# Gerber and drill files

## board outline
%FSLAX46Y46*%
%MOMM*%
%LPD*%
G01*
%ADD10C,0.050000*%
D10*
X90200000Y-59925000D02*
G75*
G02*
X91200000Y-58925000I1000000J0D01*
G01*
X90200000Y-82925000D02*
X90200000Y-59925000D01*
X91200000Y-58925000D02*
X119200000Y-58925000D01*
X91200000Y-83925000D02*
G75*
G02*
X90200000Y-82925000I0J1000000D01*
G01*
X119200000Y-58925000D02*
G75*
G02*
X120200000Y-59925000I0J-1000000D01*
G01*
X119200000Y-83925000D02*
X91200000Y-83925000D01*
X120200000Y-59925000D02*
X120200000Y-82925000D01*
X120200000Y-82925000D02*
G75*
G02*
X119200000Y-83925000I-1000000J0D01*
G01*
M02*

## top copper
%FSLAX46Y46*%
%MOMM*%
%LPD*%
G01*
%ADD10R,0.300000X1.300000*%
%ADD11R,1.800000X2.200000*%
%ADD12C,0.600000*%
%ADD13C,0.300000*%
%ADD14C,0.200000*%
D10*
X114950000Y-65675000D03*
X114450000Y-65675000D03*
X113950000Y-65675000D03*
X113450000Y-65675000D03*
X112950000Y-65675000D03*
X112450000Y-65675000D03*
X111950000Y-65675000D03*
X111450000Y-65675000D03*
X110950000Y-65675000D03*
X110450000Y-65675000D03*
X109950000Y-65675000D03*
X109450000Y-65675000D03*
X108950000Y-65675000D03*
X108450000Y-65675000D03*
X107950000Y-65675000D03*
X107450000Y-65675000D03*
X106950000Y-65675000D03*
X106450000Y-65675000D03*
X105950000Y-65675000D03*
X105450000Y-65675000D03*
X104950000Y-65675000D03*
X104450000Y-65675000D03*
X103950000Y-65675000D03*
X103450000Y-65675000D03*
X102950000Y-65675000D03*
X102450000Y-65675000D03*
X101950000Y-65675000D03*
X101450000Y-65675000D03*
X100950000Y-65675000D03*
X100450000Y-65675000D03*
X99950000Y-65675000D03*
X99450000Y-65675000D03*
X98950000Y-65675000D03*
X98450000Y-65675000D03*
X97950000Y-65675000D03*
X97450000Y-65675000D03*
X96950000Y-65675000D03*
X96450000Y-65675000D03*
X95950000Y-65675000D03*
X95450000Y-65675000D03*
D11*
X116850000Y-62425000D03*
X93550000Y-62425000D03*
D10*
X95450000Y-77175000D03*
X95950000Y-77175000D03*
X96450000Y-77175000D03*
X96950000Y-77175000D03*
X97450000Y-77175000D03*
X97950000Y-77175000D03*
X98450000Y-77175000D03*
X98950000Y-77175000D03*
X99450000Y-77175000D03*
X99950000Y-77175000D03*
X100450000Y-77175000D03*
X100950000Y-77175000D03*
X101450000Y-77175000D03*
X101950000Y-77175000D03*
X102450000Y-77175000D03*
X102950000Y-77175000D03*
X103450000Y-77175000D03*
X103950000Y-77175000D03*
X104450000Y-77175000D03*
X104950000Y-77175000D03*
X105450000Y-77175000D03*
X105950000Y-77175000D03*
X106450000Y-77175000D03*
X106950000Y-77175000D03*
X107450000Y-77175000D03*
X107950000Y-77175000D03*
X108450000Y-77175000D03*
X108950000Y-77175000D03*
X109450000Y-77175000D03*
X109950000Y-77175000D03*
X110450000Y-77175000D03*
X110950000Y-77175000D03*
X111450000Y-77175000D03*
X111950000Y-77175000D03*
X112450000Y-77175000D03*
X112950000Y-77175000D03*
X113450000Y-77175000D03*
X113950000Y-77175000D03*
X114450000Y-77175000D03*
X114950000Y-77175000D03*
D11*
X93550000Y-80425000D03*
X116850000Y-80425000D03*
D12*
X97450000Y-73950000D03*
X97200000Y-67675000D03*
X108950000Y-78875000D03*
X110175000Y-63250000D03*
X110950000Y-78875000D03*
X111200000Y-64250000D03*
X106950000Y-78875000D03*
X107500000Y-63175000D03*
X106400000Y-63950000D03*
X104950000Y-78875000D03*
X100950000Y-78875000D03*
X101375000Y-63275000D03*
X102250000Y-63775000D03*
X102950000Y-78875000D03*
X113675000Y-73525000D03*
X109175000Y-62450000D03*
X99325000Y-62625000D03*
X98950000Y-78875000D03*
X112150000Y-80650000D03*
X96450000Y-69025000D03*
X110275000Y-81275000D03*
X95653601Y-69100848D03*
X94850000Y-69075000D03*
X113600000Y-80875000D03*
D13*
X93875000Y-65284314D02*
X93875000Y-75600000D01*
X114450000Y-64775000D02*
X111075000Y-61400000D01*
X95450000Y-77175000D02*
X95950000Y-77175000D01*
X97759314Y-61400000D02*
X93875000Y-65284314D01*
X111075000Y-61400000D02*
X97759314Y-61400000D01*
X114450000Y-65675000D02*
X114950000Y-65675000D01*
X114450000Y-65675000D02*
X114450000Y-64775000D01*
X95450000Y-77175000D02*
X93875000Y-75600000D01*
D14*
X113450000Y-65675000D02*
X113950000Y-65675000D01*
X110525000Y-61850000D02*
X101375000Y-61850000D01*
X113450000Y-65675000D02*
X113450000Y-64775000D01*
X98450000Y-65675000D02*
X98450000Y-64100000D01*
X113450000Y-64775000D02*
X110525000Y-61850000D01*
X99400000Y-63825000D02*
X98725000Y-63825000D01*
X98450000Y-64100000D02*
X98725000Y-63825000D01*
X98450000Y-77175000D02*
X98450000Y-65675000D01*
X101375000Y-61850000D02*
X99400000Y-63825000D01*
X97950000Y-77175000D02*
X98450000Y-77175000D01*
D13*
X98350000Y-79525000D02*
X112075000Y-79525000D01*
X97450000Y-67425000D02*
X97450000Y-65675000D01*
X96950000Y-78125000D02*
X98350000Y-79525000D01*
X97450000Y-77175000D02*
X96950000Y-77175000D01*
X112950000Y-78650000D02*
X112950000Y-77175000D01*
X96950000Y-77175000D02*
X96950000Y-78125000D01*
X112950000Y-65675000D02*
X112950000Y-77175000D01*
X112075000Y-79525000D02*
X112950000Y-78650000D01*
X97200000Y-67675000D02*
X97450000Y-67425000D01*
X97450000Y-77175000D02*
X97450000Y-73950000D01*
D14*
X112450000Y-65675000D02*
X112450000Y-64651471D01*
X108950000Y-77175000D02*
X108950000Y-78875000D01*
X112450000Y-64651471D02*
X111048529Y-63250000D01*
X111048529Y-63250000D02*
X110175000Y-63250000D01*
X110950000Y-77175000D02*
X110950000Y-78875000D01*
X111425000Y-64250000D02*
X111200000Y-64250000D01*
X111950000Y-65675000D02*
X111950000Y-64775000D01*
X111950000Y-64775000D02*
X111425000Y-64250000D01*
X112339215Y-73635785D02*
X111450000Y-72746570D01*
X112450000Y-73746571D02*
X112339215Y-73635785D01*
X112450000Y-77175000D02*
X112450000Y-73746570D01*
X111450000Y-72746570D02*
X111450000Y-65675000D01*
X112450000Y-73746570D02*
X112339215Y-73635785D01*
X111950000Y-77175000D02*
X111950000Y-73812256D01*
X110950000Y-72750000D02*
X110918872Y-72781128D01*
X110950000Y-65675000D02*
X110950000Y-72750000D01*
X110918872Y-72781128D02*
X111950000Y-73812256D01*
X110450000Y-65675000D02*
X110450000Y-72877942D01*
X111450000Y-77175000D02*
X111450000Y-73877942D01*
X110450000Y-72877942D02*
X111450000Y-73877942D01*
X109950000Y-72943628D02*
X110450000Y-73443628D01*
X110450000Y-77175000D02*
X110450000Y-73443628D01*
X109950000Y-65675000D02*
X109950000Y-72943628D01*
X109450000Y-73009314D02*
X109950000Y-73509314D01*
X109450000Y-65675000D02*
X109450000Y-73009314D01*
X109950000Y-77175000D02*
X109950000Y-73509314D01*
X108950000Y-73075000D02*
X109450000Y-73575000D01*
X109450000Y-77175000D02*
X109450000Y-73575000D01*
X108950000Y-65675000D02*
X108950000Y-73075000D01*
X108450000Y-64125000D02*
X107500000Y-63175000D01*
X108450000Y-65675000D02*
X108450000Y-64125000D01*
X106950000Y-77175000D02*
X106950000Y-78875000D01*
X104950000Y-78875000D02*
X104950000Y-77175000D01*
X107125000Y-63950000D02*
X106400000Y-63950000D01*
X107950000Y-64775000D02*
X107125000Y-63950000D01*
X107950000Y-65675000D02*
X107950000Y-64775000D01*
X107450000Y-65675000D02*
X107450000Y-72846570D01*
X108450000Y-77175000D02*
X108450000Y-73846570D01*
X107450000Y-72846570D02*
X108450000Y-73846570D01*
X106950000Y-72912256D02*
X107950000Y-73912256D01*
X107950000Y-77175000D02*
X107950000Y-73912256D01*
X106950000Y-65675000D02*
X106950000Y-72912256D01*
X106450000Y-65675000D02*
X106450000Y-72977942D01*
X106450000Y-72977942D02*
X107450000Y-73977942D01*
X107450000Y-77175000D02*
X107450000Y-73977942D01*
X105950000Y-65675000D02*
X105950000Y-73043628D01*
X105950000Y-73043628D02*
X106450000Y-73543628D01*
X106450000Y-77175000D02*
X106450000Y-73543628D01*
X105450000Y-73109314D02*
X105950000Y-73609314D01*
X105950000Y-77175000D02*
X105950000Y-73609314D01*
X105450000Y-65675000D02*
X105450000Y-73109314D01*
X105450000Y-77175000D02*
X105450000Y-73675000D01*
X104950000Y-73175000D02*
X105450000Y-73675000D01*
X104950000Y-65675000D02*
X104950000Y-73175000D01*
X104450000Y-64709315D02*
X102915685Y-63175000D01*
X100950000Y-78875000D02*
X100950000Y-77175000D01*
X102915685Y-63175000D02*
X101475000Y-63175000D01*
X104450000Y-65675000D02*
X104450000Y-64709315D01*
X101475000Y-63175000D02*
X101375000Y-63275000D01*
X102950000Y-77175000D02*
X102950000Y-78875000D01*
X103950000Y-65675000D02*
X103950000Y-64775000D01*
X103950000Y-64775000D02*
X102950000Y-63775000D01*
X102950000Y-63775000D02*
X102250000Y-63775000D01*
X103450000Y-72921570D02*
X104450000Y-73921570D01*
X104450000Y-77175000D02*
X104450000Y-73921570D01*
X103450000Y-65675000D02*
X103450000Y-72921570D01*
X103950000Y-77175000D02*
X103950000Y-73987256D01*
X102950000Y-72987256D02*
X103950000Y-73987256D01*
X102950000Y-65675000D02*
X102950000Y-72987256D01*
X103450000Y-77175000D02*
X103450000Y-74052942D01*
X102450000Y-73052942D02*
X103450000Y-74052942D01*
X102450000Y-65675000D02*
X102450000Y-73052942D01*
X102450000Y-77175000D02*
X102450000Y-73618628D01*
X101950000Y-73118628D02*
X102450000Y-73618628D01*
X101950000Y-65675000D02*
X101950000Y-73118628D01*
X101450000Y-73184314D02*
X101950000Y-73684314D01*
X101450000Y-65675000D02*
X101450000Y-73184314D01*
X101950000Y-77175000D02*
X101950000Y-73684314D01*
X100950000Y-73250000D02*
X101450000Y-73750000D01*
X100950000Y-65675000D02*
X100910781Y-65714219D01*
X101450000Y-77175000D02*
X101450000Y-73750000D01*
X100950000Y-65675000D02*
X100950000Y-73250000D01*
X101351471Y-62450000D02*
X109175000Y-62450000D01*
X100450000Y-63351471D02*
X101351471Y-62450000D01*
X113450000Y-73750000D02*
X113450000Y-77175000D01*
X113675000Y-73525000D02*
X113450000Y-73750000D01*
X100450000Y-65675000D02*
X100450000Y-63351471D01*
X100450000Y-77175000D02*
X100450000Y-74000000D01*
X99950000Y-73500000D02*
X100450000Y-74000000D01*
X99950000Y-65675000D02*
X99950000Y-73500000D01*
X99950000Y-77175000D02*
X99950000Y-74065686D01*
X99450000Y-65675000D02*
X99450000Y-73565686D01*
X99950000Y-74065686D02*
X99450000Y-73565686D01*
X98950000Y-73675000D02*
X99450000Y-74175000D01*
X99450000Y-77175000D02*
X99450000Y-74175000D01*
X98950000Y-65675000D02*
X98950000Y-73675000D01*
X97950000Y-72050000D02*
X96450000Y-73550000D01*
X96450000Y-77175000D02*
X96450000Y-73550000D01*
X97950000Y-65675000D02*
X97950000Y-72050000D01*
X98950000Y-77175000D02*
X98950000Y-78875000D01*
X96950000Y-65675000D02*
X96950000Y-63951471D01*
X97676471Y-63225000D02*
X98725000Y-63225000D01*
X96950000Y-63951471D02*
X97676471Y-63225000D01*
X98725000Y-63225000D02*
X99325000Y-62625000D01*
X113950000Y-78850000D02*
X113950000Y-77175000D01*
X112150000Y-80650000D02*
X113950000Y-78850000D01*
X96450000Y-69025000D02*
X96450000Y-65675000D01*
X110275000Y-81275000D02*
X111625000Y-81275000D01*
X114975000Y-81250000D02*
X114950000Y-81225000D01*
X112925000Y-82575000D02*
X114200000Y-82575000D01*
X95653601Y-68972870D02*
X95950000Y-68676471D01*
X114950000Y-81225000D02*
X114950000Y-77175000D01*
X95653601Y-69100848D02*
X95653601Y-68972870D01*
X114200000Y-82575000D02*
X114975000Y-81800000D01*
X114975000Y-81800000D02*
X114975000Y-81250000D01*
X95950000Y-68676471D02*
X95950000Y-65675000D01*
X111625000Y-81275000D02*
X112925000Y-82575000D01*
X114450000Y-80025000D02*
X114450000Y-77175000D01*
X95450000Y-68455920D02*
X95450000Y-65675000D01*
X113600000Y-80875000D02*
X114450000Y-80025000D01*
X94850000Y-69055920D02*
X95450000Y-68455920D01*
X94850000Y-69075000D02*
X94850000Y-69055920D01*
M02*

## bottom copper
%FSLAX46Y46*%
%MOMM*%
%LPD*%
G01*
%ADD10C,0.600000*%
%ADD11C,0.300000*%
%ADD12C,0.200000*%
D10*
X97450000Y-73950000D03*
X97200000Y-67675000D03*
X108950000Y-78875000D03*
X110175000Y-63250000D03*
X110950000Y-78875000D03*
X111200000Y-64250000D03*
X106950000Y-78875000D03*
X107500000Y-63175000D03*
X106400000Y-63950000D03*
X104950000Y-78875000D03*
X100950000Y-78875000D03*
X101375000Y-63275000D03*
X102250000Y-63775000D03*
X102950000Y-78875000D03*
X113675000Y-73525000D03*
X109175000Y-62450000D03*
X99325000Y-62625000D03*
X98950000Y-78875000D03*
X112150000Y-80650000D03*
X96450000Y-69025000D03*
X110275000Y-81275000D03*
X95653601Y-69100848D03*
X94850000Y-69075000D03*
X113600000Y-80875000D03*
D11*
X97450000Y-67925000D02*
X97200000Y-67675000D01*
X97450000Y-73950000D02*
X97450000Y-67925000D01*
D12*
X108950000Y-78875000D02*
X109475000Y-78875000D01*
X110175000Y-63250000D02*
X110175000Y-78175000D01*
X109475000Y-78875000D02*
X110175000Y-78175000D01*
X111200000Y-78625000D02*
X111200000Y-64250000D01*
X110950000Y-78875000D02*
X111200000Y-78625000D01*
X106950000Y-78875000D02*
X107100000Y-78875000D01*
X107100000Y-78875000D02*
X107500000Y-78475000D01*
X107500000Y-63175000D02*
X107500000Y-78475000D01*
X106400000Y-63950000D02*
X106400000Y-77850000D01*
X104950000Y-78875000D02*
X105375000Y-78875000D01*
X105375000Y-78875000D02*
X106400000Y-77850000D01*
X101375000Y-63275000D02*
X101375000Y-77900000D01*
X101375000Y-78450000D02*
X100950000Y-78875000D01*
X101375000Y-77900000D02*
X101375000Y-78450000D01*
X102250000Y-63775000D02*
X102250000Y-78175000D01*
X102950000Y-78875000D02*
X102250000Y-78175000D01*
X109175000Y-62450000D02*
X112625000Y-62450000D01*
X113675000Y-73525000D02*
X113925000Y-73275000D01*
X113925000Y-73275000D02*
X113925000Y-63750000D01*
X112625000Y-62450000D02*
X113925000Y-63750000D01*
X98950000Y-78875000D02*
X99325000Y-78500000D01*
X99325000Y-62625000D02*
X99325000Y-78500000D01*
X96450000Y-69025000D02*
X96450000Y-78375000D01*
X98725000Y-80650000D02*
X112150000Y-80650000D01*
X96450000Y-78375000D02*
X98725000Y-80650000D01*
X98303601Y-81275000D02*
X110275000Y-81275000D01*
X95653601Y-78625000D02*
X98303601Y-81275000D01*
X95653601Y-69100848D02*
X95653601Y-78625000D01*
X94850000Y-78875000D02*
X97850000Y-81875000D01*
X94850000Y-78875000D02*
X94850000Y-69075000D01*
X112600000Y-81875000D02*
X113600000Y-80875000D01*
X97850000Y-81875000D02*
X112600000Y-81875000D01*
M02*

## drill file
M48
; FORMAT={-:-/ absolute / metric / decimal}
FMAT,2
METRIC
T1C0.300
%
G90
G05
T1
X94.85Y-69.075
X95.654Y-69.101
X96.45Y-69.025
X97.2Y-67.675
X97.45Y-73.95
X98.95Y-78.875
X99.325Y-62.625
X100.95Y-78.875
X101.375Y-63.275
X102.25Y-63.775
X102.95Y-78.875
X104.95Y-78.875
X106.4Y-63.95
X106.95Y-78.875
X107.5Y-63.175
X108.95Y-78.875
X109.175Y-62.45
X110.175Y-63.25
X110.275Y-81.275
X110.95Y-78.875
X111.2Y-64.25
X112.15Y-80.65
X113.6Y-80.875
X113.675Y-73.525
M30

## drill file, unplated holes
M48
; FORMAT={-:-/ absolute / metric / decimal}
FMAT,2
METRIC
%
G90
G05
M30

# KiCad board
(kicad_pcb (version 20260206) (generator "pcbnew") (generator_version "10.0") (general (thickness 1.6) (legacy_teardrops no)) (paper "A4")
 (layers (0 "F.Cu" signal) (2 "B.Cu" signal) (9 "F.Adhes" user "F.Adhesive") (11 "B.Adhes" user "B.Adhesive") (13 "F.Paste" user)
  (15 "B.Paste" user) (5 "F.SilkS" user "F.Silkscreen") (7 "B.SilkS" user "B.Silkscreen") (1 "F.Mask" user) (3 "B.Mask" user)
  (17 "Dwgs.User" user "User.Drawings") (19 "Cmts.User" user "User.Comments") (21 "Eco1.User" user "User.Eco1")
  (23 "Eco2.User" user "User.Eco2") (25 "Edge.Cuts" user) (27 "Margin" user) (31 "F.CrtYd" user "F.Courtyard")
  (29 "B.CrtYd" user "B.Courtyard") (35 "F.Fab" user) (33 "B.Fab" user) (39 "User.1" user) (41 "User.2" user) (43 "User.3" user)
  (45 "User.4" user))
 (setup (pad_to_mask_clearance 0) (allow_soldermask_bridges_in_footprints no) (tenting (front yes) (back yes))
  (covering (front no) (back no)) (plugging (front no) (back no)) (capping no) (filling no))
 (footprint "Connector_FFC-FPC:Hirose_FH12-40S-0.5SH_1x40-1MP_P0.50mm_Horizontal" (layer "F.Cu") (at 105.2 63.825 180)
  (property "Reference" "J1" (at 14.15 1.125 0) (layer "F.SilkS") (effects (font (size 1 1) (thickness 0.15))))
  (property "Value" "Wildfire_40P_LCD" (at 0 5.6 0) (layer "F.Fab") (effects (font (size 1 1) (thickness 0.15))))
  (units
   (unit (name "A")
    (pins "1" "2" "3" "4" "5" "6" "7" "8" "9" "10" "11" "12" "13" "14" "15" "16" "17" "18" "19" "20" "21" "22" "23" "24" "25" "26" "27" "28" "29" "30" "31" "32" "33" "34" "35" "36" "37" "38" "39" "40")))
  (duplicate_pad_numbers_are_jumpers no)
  (pad "1" smd rect (at -9.75 -1.85 180) (size 0.3 1.3) (layers "F.Cu" "F.Mask" "F.Paste") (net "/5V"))
  (pad "2" smd rect (at -9.25 -1.85 180) (size 0.3 1.3) (layers "F.Cu" "F.Mask" "F.Paste") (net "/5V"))
  (pad "3" smd rect (at -8.75 -1.85 180) (size 0.3 1.3) (layers "F.Cu" "F.Mask" "F.Paste") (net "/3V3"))
  (pad "4" smd rect (at -8.25 -1.85 180) (size 0.3 1.3) (layers "F.Cu" "F.Mask" "F.Paste") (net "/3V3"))
  (pad "5" smd rect (at -7.75 -1.85 180) (size 0.3 1.3) (layers "F.Cu" "F.Mask" "F.Paste") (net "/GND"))
  (pad "6" smd rect (at -7.25 -1.85 180) (size 0.3 1.3) (layers "F.Cu" "F.Mask" "F.Paste") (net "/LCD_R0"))
  (pad "7" smd rect (at -6.75 -1.85 180) (size 0.3 1.3) (layers "F.Cu" "F.Mask" "F.Paste") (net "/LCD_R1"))
  (pad "8" smd rect (at -6.25 -1.85 180) (size 0.3 1.3) (layers "F.Cu" "F.Mask" "F.Paste") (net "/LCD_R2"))
  (pad "9" smd rect (at -5.75 -1.85 180) (size 0.3 1.3) (layers "F.Cu" "F.Mask" "F.Paste") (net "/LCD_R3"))
  (pad "10" smd rect (at -5.25 -1.85 180) (size 0.3 1.3) (layers "F.Cu" "F.Mask" "F.Paste") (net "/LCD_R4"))
  (pad "11" smd rect (at -4.75 -1.85 180) (size 0.3 1.3) (layers "F.Cu" "F.Mask" "F.Paste") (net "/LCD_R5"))
  (pad "12" smd rect (at -4.25 -1.85 180) (size 0.3 1.3) (layers "F.Cu" "F.Mask" "F.Paste") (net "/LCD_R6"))
  (pad "13" smd rect (at -3.75 -1.85 180) (size 0.3 1.3) (layers "F.Cu" "F.Mask" "F.Paste") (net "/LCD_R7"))
  (pad "14" smd rect (at -3.25 -1.85 180) (size 0.3 1.3) (layers "F.Cu" "F.Mask" "F.Paste") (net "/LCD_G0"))
  (pad "15" smd rect (at -2.75 -1.85 180) (size 0.3 1.3) (layers "F.Cu" "F.Mask" "F.Paste") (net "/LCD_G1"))
  (pad "16" smd rect (at -2.25 -1.85 180) (size 0.3 1.3) (layers "F.Cu" "F.Mask" "F.Paste") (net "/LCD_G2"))
  (pad "17" smd rect (at -1.75 -1.85 180) (size 0.3 1.3) (layers "F.Cu" "F.Mask" "F.Paste") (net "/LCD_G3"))
  (pad "18" smd rect (at -1.25 -1.85 180) (size 0.3 1.3) (layers "F.Cu" "F.Mask" "F.Paste") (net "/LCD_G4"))
  (pad "19" smd rect (at -0.75 -1.85 180) (size 0.3 1.3) (layers "F.Cu" "F.Mask" "F.Paste") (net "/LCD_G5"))
  (pad "20" smd rect (at -0.25 -1.85 180) (size 0.3 1.3) (layers "F.Cu" "F.Mask" "F.Paste") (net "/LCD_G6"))
  (pad "21" smd rect (at 0.25 -1.85 180) (size 0.3 1.3) (layers "F.Cu" "F.Mask" "F.Paste") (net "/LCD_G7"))
  (pad "22" smd rect (at 0.75 -1.85 180) (size 0.3 1.3) (layers "F.Cu" "F.Mask" "F.Paste") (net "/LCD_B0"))
  (pad "23" smd rect (at 1.25 -1.85 180) (size 0.3 1.3) (layers "F.Cu" "F.Mask" "F.Paste") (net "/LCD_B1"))
  (pad "24" smd rect (at 1.75 -1.85 180) (size 0.3 1.3) (layers "F.Cu" "F.Mask" "F.Paste") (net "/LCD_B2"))
  (pad "25" smd rect (at 2.25 -1.85 180) (size 0.3 1.3) (layers "F.Cu" "F.Mask" "F.Paste") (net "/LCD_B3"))
  (pad "26" smd rect (at 2.75 -1.85 180) (size 0.3 1.3) (layers "F.Cu" "F.Mask" "F.Paste") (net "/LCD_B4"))
  (pad "27" smd rect (at 3.25 -1.85 180) (size 0.3 1.3) (layers "F.Cu" "F.Mask" "F.Paste") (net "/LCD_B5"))
  (pad "28" smd rect (at 3.75 -1.85 180) (size 0.3 1.3) (layers "F.Cu" "F.Mask" "F.Paste") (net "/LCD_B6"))
  (pad "29" smd rect (at 4.25 -1.85 180) (size 0.3 1.3) (layers "F.Cu" "F.Mask" "F.Paste") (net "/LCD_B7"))
  (pad "30" smd rect (at 4.75 -1.85 180) (size 0.3 1.3) (layers "F.Cu" "F.Mask" "F.Paste") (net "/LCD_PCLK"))
  (pad "31" smd rect (at 5.25 -1.85 180) (size 0.3 1.3) (layers "F.Cu" "F.Mask" "F.Paste") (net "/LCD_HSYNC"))
  (pad "32" smd rect (at 5.75 -1.85 180) (size 0.3 1.3) (layers "F.Cu" "F.Mask" "F.Paste") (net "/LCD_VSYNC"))
  (pad "33" smd rect (at 6.25 -1.85 180) (size 0.3 1.3) (layers "F.Cu" "F.Mask" "F.Paste") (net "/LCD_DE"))
  (pad "34" smd rect (at 6.75 -1.85 180) (size 0.3 1.3) (layers "F.Cu" "F.Mask" "F.Paste") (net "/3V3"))
  (pad "35" smd rect (at 7.25 -1.85 180) (size 0.3 1.3) (layers "F.Cu" "F.Mask" "F.Paste") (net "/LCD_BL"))
  (pad "36" smd rect (at 7.75 -1.85 180) (size 0.3 1.3) (layers "F.Cu" "F.Mask" "F.Paste") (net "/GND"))
  (pad "37" smd rect (at 8.25 -1.85 180) (size 0.3 1.3) (layers "F.Cu" "F.Mask" "F.Paste") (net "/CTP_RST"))
  (pad "38" smd rect (at 8.75 -1.85 180) (size 0.3 1.3) (layers "F.Cu" "F.Mask" "F.Paste") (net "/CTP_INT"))
  (pad "39" smd rect (at 9.25 -1.85 180) (size 0.3 1.3) (layers "F.Cu" "F.Mask" "F.Paste") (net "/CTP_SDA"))
  (pad "40" smd rect (at 9.75 -1.85 180) (size 0.3 1.3) (layers "F.Cu" "F.Mask" "F.Paste") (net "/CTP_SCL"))
  (pad "MP" smd rect (at -11.65 1.4 180) (size 1.8 2.2) (layers "F.Cu" "F.Mask" "F.Paste"))
  (pad "MP" smd rect (at 11.65 1.4 180) (size 1.8 2.2) (layers "F.Cu" "F.Mask" "F.Paste")))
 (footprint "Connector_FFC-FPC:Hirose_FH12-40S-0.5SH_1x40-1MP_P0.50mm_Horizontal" (layer "F.Cu") (at 105.2 79.025)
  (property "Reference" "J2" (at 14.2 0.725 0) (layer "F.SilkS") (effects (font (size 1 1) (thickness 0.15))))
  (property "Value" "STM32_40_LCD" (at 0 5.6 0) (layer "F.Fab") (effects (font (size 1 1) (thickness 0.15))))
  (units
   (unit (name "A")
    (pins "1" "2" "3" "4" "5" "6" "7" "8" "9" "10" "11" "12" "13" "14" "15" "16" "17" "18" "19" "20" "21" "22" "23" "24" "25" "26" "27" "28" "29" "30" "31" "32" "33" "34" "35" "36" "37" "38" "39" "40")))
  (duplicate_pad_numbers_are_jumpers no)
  (pad "1" smd rect (at -9.75 -1.85) (size 0.3 1.3) (layers "F.Cu" "F.Mask" "F.Paste") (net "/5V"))
  (pad "2" smd rect (at -9.25 -1.85) (size 0.3 1.3) (layers "F.Cu" "F.Mask" "F.Paste") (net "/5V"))
  (pad "3" smd rect (at -8.75 -1.85) (size 0.3 1.3) (layers "F.Cu" "F.Mask" "F.Paste") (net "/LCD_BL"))
  (pad "4" smd rect (at -8.25 -1.85) (size 0.3 1.3) (layers "F.Cu" "F.Mask" "F.Paste") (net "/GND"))
  (pad "5" smd rect (at -7.75 -1.85) (size 0.3 1.3) (layers "F.Cu" "F.Mask" "F.Paste") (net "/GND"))
  (pad "6" smd rect (at -7.25 -1.85) (size 0.3 1.3) (layers "F.Cu" "F.Mask" "F.Paste") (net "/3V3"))
  (pad "7" smd rect (at -6.75 -1.85) (size 0.3 1.3) (layers "F.Cu" "F.Mask" "F.Paste") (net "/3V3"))
  (pad "8" smd rect (at -6.25 -1.85) (size 0.3 1.3) (layers "F.Cu" "F.Mask" "F.Paste") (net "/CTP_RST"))
  (pad "9" smd rect (at -5.75 -1.85) (size 0.3 1.3) (layers "F.Cu" "F.Mask" "F.Paste") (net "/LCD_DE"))
  (pad "10" smd rect (at -5.25 -1.85) (size 0.3 1.3) (layers "F.Cu" "F.Mask" "F.Paste") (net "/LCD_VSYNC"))
  (pad "11" smd rect (at -4.75 -1.85) (size 0.3 1.3) (layers "F.Cu" "F.Mask" "F.Paste") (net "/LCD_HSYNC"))
  (pad "12" smd rect (at -4.25 -1.85) (size 0.3 1.3) (layers "F.Cu" "F.Mask" "F.Paste") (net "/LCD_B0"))
  (pad "13" smd rect (at -3.75 -1.85) (size 0.3 1.3) (layers "F.Cu" "F.Mask" "F.Paste") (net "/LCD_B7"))
  (pad "14" smd rect (at -3.25 -1.85) (size 0.3 1.3) (layers "F.Cu" "F.Mask" "F.Paste") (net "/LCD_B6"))
  (pad "15" smd rect (at -2.75 -1.85) (size 0.3 1.3) (layers "F.Cu" "F.Mask" "F.Paste") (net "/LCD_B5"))
  (pad "16" smd rect (at -2.25 -1.85) (size 0.3 1.3) (layers "F.Cu" "F.Mask" "F.Paste") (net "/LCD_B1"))
  (pad "17" smd rect (at -1.75 -1.85) (size 0.3 1.3) (layers "F.Cu" "F.Mask" "F.Paste") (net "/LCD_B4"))
  (pad "18" smd rect (at -1.25 -1.85) (size 0.3 1.3) (layers "F.Cu" "F.Mask" "F.Paste") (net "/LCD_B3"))
  (pad "19" smd rect (at -0.75 -1.85) (size 0.3 1.3) (layers "F.Cu" "F.Mask" "F.Paste") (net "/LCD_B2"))
  (pad "20" smd rect (at -0.25 -1.85) (size 0.3 1.3) (layers "F.Cu" "F.Mask" "F.Paste") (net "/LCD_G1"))
  (pad "21" smd rect (at 0.25 -1.85) (size 0.3 1.3) (layers "F.Cu" "F.Mask" "F.Paste") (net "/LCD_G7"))
  (pad "22" smd rect (at 0.75 -1.85) (size 0.3 1.3) (layers "F.Cu" "F.Mask" "F.Paste") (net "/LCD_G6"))
  (pad "23" smd rect (at 1.25 -1.85) (size 0.3 1.3) (layers "F.Cu" "F.Mask" "F.Paste") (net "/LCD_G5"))
  (pad "24" smd rect (at 1.75 -1.85) (size 0.3 1.3) (layers "F.Cu" "F.Mask" "F.Paste") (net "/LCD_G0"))
  (pad "25" smd rect (at 2.25 -1.85) (size 0.3 1.3) (layers "F.Cu" "F.Mask" "F.Paste") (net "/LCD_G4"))
  (pad "26" smd rect (at 2.75 -1.85) (size 0.3 1.3) (layers "F.Cu" "F.Mask" "F.Paste") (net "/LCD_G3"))
  (pad "27" smd rect (at 3.25 -1.85) (size 0.3 1.3) (layers "F.Cu" "F.Mask" "F.Paste") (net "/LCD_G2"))
  (pad "28" smd rect (at 3.75 -1.85) (size 0.3 1.3) (layers "F.Cu" "F.Mask" "F.Paste") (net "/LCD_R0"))
  (pad "29" smd rect (at 4.25 -1.85) (size 0.3 1.3) (layers "F.Cu" "F.Mask" "F.Paste") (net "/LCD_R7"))
  (pad "30" smd rect (at 4.75 -1.85) (size 0.3 1.3) (layers "F.Cu" "F.Mask" "F.Paste") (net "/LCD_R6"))
  (pad "31" smd rect (at 5.25 -1.85) (size 0.3 1.3) (layers "F.Cu" "F.Mask" "F.Paste") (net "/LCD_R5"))
  (pad "32" smd rect (at 5.75 -1.85) (size 0.3 1.3) (layers "F.Cu" "F.Mask" "F.Paste") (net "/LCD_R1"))
  (pad "33" smd rect (at 6.25 -1.85) (size 0.3 1.3) (layers "F.Cu" "F.Mask" "F.Paste") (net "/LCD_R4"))
  (pad "34" smd rect (at 6.75 -1.85) (size 0.3 1.3) (layers "F.Cu" "F.Mask" "F.Paste") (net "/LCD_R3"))
  (pad "35" smd rect (at 7.25 -1.85) (size 0.3 1.3) (layers "F.Cu" "F.Mask" "F.Paste") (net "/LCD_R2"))
  (pad "36" smd rect (at 7.75 -1.85) (size 0.3 1.3) (layers "F.Cu" "F.Mask" "F.Paste") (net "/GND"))
  (pad "37" smd rect (at 8.25 -1.85) (size 0.3 1.3) (layers "F.Cu" "F.Mask" "F.Paste") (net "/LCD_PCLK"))
  (pad "38" smd rect (at 8.75 -1.85) (size 0.3 1.3) (layers "F.Cu" "F.Mask" "F.Paste") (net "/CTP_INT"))
  (pad "39" smd rect (at 9.25 -1.85) (size 0.3 1.3) (layers "F.Cu" "F.Mask" "F.Paste") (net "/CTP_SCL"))
  (pad "40" smd rect (at 9.75 -1.85) (size 0.3 1.3) (layers "F.Cu" "F.Mask" "F.Paste") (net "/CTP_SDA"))
  (pad "MP" smd rect (at -11.65 1.4) (size 1.8 2.2) (layers "F.Cu" "F.Mask" "F.Paste"))
  (pad "MP" smd rect (at 11.65 1.4) (size 1.8 2.2) (layers "F.Cu" "F.Mask" "F.Paste")))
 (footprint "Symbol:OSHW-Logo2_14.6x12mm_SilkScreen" (layer "B.Cu") (at 105.200001 71.411466 180)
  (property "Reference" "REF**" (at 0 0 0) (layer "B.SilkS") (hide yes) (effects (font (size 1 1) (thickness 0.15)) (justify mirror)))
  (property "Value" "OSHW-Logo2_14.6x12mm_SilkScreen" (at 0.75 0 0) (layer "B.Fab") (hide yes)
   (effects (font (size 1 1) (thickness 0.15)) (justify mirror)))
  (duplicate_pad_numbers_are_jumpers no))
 (gr_arc (start 90.2 59.925) (mid 90.492893 59.217893) (end 91.2 58.925) (stroke (width 0.05) (type default)) (layer "Edge.Cuts"))
 (gr_line (start 90.2 82.925) (end 90.2 59.925) (stroke (width 0.05) (type default)) (layer "Edge.Cuts"))
 (gr_line (start 91.2 58.925) (end 119.2 58.925) (stroke (width 0.05) (type default)) (layer "Edge.Cuts"))
 (gr_arc (start 91.2 83.925) (mid 90.492893 83.632107) (end 90.2 82.925) (stroke (width 0.05) (type default)) (layer "Edge.Cuts"))
 (gr_arc (start 119.2 58.925) (mid 119.907107 59.217893) (end 120.2 59.925) (stroke (width 0.05) (type default)) (layer "Edge.Cuts"))
 (gr_line (start 119.2 83.925) (end 91.2 83.925) (stroke (width 0.05) (type default)) (layer "Edge.Cuts"))
 (gr_line (start 120.2 59.925) (end 120.2 82.925) (stroke (width 0.05) (type default)) (layer "Edge.Cuts"))
 (gr_arc (start 120.2 82.925) (mid 119.907107 83.632107) (end 119.2 83.925) (stroke (width 0.05) (type default)) (layer "Edge.Cuts"))
 (segment (start 93.875 65.284314) (end 93.875 75.6) (width 0.3) (layer "F.Cu") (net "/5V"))
 (segment (start 114.45 64.775) (end 111.075 61.4) (width 0.3) (layer "F.Cu") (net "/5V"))
 (segment (start 95.45 77.175) (end 95.95 77.175) (width 0.3) (layer "F.Cu") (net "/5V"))
 (segment (start 97.759314 61.4) (end 93.875 65.284314) (width 0.3) (layer "F.Cu") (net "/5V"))
 (segment (start 111.075 61.4) (end 97.759314 61.4) (width 0.3) (layer "F.Cu") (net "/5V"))
 (segment (start 114.45 65.675) (end 114.95 65.675) (width 0.3) (layer "F.Cu") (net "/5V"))
 (segment (start 114.45 65.675) (end 114.45 64.775) (width 0.3) (layer "F.Cu") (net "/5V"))
 (segment (start 95.45 77.175) (end 93.875 75.6) (width 0.3) (layer "F.Cu") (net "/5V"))
 (segment (start 113.45 65.675) (end 113.95 65.675) (width 0.2) (layer "F.Cu") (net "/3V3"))
 (segment (start 110.525 61.85) (end 101.375 61.85) (width 0.2) (layer "F.Cu") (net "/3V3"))
 (segment (start 113.45 65.675) (end 113.45 64.775) (width 0.2) (layer "F.Cu") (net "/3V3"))
 (segment (start 98.45 65.675) (end 98.45 64.1) (width 0.2) (layer "F.Cu") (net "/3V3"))
 (segment (start 113.45 64.775) (end 110.525 61.85) (width 0.2) (layer "F.Cu") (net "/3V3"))
 (segment (start 99.4 63.825) (end 98.725 63.825) (width 0.2) (layer "F.Cu") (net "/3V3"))
 (segment (start 98.45 64.1) (end 98.725 63.825) (width 0.2) (layer "F.Cu") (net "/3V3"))
 (segment (start 98.45 77.175) (end 98.45 65.675) (width 0.2) (layer "F.Cu") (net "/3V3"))
 (segment (start 101.375 61.85) (end 99.4 63.825) (width 0.2) (layer "F.Cu") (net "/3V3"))
 (segment (start 97.95 77.175) (end 98.45 77.175) (width 0.2) (layer "F.Cu") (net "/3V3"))
 (segment (start 98.35 79.525) (end 112.075 79.525) (width 0.3) (layer "F.Cu") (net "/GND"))
 (segment (start 97.45 67.425) (end 97.45 65.675) (width 0.3) (layer "F.Cu") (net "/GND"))
 (segment (start 96.95 78.125) (end 98.35 79.525) (width 0.3) (layer "F.Cu") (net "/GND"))
 (segment (start 97.45 77.175) (end 96.95 77.175) (width 0.3) (layer "F.Cu") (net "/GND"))
 (segment (start 112.95 78.65) (end 112.95 77.175) (width 0.3) (layer "F.Cu") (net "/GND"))
 (segment (start 96.95 77.175) (end 96.95 78.125) (width 0.3) (layer "F.Cu") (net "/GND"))
 (segment (start 112.95 65.675) (end 112.95 77.175) (width 0.3) (layer "F.Cu") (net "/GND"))
 (segment (start 112.075 79.525) (end 112.95 78.65) (width 0.3) (layer "F.Cu") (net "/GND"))
 (segment (start 97.2 67.675) (end 97.45 67.425) (width 0.3) (layer "F.Cu") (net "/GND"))
 (segment (start 97.45 77.175) (end 97.45 73.95) (width 0.3) (layer "F.Cu") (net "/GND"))
 (via (at 97.45 73.95) (size 0.6) (drill 0.3) (layers "F.Cu" "B.Cu") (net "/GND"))
 (via (at 97.2 67.675) (size 0.6) (drill 0.3) (layers "F.Cu" "B.Cu") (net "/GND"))
 (segment (start 97.45 67.925) (end 97.2 67.675) (width 0.3) (layer "B.Cu") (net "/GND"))
 (segment (start 97.45 73.95) (end 97.45 67.925) (width 0.3) (layer "B.Cu") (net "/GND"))
 (segment (start 112.45 65.675) (end 112.45 64.651471) (width 0.2) (layer "F.Cu") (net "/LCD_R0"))
 (segment (start 108.95 77.175) (end 108.95 78.875) (width 0.2) (layer "F.Cu") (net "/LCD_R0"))
 (segment (start 112.45 64.651471) (end 111.048529 63.25) (width 0.2) (layer "F.Cu") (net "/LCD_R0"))
 (segment (start 111.048529 63.25) (end 110.175 63.25) (width 0.2) (layer "F.Cu") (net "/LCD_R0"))
 (via (at 108.95 78.875) (size 0.6) (drill 0.3) (layers "F.Cu" "B.Cu") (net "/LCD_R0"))
 (via (at 110.175 63.25) (size 0.6) (drill 0.3) (layers "F.Cu" "B.Cu") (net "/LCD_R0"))
 (segment (start 108.95 78.875) (end 109.475 78.875) (width 0.2) (layer "B.Cu") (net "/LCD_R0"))
 (segment (start 110.175 63.25) (end 110.175 78.175) (width 0.2) (layer "B.Cu") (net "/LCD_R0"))
 (segment (start 109.475 78.875) (end 110.175 78.175) (width 0.2) (layer "B.Cu") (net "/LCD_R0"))
 (segment (start 110.95 77.175) (end 110.95 78.875) (width 0.2) (layer "F.Cu") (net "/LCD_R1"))
 (segment (start 111.425 64.25) (end 111.2 64.25) (width 0.2) (layer "F.Cu") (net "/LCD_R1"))
 (segment (start 111.95 65.675) (end 111.95 64.775) (width 0.2) (layer "F.Cu") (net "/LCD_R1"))
 (segment (start 111.95 64.775) (end 111.425 64.25) (width 0.2) (layer "F.Cu") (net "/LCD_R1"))
 (via (at 110.95 78.875) (size 0.6) (drill 0.3) (layers "F.Cu" "B.Cu") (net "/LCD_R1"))
 (via (at 111.2 64.25) (size 0.6) (drill 0.3) (layers "F.Cu" "B.Cu") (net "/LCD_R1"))
 (segment (start 111.2 78.625) (end 111.2 64.25) (width 0.2) (layer "B.Cu") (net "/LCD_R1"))
 (segment (start 110.95 78.875) (end 111.2 78.625) (width 0.2) (layer "B.Cu") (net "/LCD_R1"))
 (segment (start 112.339215 73.635785) (end 111.45 72.74657) (width 0.2) (layer "F.Cu") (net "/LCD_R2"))
 (segment (start 112.45 73.746571) (end 112.339215 73.635785) (width 0.2) (layer "F.Cu") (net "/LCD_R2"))
 (segment (start 112.45 77.175) (end 112.45 73.74657) (width 0.2) (layer "F.Cu") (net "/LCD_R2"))
 (segment (start 111.45 72.74657) (end 111.45 65.675) (width 0.2) (layer "F.Cu") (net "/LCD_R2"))
 (segment (start 112.45 73.74657) (end 112.339215 73.635785) (width 0.2) (layer "F.Cu") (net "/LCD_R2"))
 (segment (start 111.95 77.175) (end 111.95 73.812256) (width 0.2) (layer "F.Cu") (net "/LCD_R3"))
 (segment (start 110.95 72.75) (end 110.918872 72.781128) (width 0.2) (layer "F.Cu") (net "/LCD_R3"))
 (segment (start 110.95 65.675) (end 110.95 72.75) (width 0.2) (layer "F.Cu") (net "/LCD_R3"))
 (segment (start 110.918872 72.781128) (end 111.95 73.812256) (width 0.2) (layer "F.Cu") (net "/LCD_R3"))
 (segment (start 110.45 65.675) (end 110.45 72.877942) (width 0.2) (layer "F.Cu") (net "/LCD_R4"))
 (segment (start 111.45 77.175) (end 111.45 73.877942) (width 0.2) (layer "F.Cu") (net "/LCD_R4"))
 (segment (start 110.45 72.877942) (end 111.45 73.877942) (width 0.2) (layer "F.Cu") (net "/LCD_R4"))
 (segment (start 109.95 72.943628) (end 110.45 73.443628) (width 0.2) (layer "F.Cu") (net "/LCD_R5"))
 (segment (start 110.45 77.175) (end 110.45 73.443628) (width 0.2) (layer "F.Cu") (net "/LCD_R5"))
 (segment (start 109.95 65.675) (end 109.95 72.943628) (width 0.2) (layer "F.Cu") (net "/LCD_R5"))
 (segment (start 109.45 73.009314) (end 109.95 73.509314) (width 0.2) (layer "F.Cu") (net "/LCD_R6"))
 (segment (start 109.45 65.675) (end 109.45 73.009314) (width 0.2) (layer "F.Cu") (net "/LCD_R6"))
 (segment (start 109.95 77.175) (end 109.95 73.509314) (width 0.2) (layer "F.Cu") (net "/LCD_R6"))
 (segment (start 108.95 73.075) (end 109.45 73.575) (width 0.2) (layer "F.Cu") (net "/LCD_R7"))
 (segment (start 109.45 77.175) (end 109.45 73.575) (width 0.2) (layer "F.Cu") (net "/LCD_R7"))
 (segment (start 108.95 65.675) (end 108.95 73.075) (width 0.2) (layer "F.Cu") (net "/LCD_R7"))
 (segment (start 108.45 64.125) (end 107.5 63.175) (width 0.2) (layer "F.Cu") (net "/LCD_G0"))
 (segment (start 108.45 65.675) (end 108.45 64.125) (width 0.2) (layer "F.Cu") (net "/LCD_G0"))
 (segment (start 106.95 77.175) (end 106.95 78.875) (width 0.2) (layer "F.Cu") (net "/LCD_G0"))
 (via (at 106.95 78.875) (size 0.6) (drill 0.3) (layers "F.Cu" "B.Cu") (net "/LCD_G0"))
 (via (at 107.5 63.175) (size 0.6) (drill 0.3) (layers "F.Cu" "B.Cu") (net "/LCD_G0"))
 (segment (start 106.95 78.875) (end 107.1 78.875) (width 0.2) (layer "B.Cu") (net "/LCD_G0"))
 (segment (start 107.1 78.875) (end 107.5 78.475) (width 0.2) (layer "B.Cu") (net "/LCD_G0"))
 (segment (start 107.5 63.175) (end 107.5 78.475) (width 0.2) (layer "B.Cu") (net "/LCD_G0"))
 (segment (start 104.95 78.875) (end 104.95 77.175) (width 0.2) (layer "F.Cu") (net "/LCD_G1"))
 (segment (start 107.125 63.95) (end 106.4 63.95) (width 0.2) (layer "F.Cu") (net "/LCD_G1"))
 (segment (start 107.95 64.775) (end 107.125 63.95) (width 0.2) (layer "F.Cu") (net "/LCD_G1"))
 (segment (start 107.95 65.675) (end 107.95 64.775) (width 0.2) (layer "F.Cu") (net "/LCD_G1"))
 (via (at 106.4 63.95) (size 0.6) (drill 0.3) (layers "F.Cu" "B.Cu") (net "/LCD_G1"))
 (via (at 104.95 78.875) (size 0.6) (drill 0.3) (layers "F.Cu" "B.Cu") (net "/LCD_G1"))
 (segment (start 106.4 63.95) (end 106.4 77.85) (width 0.2) (layer "B.Cu") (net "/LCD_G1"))
 (segment (start 104.95 78.875) (end 105.375 78.875) (width 0.2) (layer "B.Cu") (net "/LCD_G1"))
 (segment (start 105.375 78.875) (end 106.4 77.85) (width 0.2) (layer "B.Cu") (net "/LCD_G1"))
 (segment (start 107.45 65.675) (end 107.45 72.84657) (width 0.2) (layer "F.Cu") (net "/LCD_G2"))
 (segment (start 108.45 77.175) (end 108.45 73.84657) (width 0.2) (layer "F.Cu") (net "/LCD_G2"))
 (segment (start 107.45 72.84657) (end 108.45 73.84657) (width 0.2) (layer "F.Cu") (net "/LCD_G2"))
 (segment (start 106.95 72.912256) (end 107.95 73.912256) (width 0.2) (layer "F.Cu") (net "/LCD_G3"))
 (segment (start 107.95 77.175) (end 107.95 73.912256) (width 0.2) (layer "F.Cu") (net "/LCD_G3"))
 (segment (start 106.95 65.675) (end 106.95 72.912256) (width 0.2) (layer "F.Cu") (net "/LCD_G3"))
 (segment (start 106.45 65.675) (end 106.45 72.977942) (width 0.2) (layer "F.Cu") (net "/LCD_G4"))
 (segment (start 106.45 72.977942) (end 107.45 73.977942) (width 0.2) (layer "F.Cu") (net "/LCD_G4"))
 (segment (start 107.45 77.175) (end 107.45 73.977942) (width 0.2) (layer "F.Cu") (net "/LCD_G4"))
 (segment (start 105.95 65.675) (end 105.95 73.043628) (width 0.2) (layer "F.Cu") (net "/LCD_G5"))
 (segment (start 105.95 73.043628) (end 106.45 73.543628) (width 0.2) (layer "F.Cu") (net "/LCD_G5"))
 (segment (start 106.45 77.175) (end 106.45 73.543628) (width 0.2) (layer "F.Cu") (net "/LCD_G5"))
 (segment (start 105.45 73.109314) (end 105.95 73.609314) (width 0.2) (layer "F.Cu") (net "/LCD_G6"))
 (segment (start 105.95 77.175) (end 105.95 73.609314) (width 0.2) (layer "F.Cu") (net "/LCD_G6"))
 (segment (start 105.45 65.675) (end 105.45 73.109314) (width 0.2) (layer "F.Cu") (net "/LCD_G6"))
 (segment (start 105.45 77.175) (end 105.45 73.675) (width 0.2) (layer "F.Cu") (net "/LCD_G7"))
 (segment (start 104.95 73.175) (end 105.45 73.675) (width 0.2) (layer "F.Cu") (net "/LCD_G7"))
 (segment (start 104.95 65.675) (end 104.95 73.175) (width 0.2) (layer "F.Cu") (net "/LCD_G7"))
 (segment (start 104.45 64.709315) (end 102.915685 63.175) (width 0.2) (layer "F.Cu") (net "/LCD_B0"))
 (segment (start 100.95 78.875) (end 100.95 77.175) (width 0.2) (layer "F.Cu") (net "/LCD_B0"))
 (segment (start 102.915685 63.175) (end 101.475 63.175) (width 0.2) (layer "F.Cu") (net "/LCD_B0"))
 (segment (start 104.45 65.675) (end 104.45 64.709315) (width 0.2) (layer "F.Cu") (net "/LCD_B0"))
 (segment (start 101.475 63.175) (end 101.375 63.275) (width 0.2) (layer "F.Cu") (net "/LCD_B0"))
 (via (at 100.95 78.875) (size 0.6) (drill 0.3) (layers "F.Cu" "B.Cu") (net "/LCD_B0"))
 (via (at 101.375 63.275) (size 0.6) (drill 0.3) (layers "F.Cu" "B.Cu") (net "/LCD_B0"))
 (segment (start 101.375 63.275) (end 101.375 77.9) (width 0.2) (layer "B.Cu") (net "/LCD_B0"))
 (segment (start 101.375 78.45) (end 100.95 78.875) (width 0.2) (layer "B.Cu") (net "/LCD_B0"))
 (segment (start 101.375 77.9) (end 101.375 78.45) (width 0.2) (layer "B.Cu") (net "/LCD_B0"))
 (segment (start 102.95 77.175) (end 102.95 78.875) (width 0.2) (layer "F.Cu") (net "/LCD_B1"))
 (segment (start 103.95 65.675) (end 103.95 64.775) (width 0.2) (layer "F.Cu") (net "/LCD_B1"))
 (segment (start 103.95 64.775) (end 102.95 63.775) (width 0.2) (layer "F.Cu") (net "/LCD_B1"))
 (segment (start 102.95 63.775) (end 102.25 63.775) (width 0.2) (layer "F.Cu") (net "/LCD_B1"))
 (via (at 102.25 63.775) (size 0.6) (drill 0.3) (layers "F.Cu" "B.Cu") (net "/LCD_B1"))
 (via (at 102.95 78.875) (size 0.6) (drill 0.3) (layers "F.Cu" "B.Cu") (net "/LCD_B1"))
 (segment (start 102.25 63.775) (end 102.25 78.175) (width 0.2) (layer "B.Cu") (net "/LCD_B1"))
 (segment (start 102.95 78.875) (end 102.25 78.175) (width 0.2) (layer "B.Cu") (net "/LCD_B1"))
 (segment (start 103.45 72.92157) (end 104.45 73.92157) (width 0.2) (layer "F.Cu") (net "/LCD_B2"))
 (segment (start 104.45 77.175) (end 104.45 73.92157) (width 0.2) (layer "F.Cu") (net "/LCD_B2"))
 (segment (start 103.45 65.675) (end 103.45 72.92157) (width 0.2) (layer "F.Cu") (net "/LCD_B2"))
 (segment (start 103.95 77.175) (end 103.95 73.987256) (width 0.2) (layer "F.Cu") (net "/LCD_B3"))
 (segment (start 102.95 72.987256) (end 103.95 73.987256) (width 0.2) (layer "F.Cu") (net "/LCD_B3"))
 (segment (start 102.95 65.675) (end 102.95 72.987256) (width 0.2) (layer "F.Cu") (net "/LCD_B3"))
 (segment (start 103.45 77.175) (end 103.45 74.052942) (width 0.2) (layer "F.Cu") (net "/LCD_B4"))
 (segment (start 102.45 73.052942) (end 103.45 74.052942) (width 0.2) (layer "F.Cu") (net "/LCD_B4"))
 (segment (start 102.45 65.675) (end 102.45 73.052942) (width 0.2) (layer "F.Cu") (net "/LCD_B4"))
 (segment (start 102.45 77.175) (end 102.45 73.618628) (width 0.2) (layer "F.Cu") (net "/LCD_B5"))
 (segment (start 101.95 73.118628) (end 102.45 73.618628) (width 0.2) (layer "F.Cu") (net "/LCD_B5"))
 (segment (start 101.95 65.675) (end 101.95 73.118628) (width 0.2) (layer "F.Cu") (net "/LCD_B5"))
 (segment (start 101.45 73.184314) (end 101.95 73.684314) (width 0.2) (layer "F.Cu") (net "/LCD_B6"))
 (segment (start 101.45 65.675) (end 101.45 73.184314) (width 0.2) (layer "F.Cu") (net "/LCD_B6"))
 (segment (start 101.95 77.175) (end 101.95 73.684314) (width 0.2) (layer "F.Cu") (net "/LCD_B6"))
 (segment (start 100.95 73.25) (end 101.45 73.75) (width 0.2) (layer "F.Cu") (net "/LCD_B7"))
 (segment (start 100.95 65.675) (end 100.910781 65.714219) (width 0.2) (layer "F.Cu") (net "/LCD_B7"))
 (segment (start 101.45 77.175) (end 101.45 73.75) (width 0.2) (layer "F.Cu") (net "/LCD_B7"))
 (segment (start 100.95 65.675) (end 100.95 73.25) (width 0.2) (layer "F.Cu") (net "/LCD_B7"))
 (segment (start 101.351471 62.45) (end 109.175 62.45) (width 0.2) (layer "F.Cu") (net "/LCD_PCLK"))
 (segment (start 100.45 63.351471) (end 101.351471 62.45) (width 0.2) (layer "F.Cu") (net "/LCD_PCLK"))
 (segment (start 113.45 73.75) (end 113.45 77.175) (width 0.2) (layer "F.Cu") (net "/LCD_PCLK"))
 (segment (start 113.675 73.525) (end 113.45 73.75) (width 0.2) (layer "F.Cu") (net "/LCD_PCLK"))
 (segment (start 100.45 65.675) (end 100.45 63.351471) (width 0.2) (layer "F.Cu") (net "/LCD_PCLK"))
 (via (at 113.675 73.525) (size 0.6) (drill 0.3) (layers "F.Cu" "B.Cu") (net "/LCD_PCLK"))
 (via (at 109.175 62.45) (size 0.6) (drill 0.3) (layers "F.Cu" "B.Cu") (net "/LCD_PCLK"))
 (segment (start 109.175 62.45) (end 112.625 62.45) (width 0.2) (layer "B.Cu") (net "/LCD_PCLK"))
 (segment (start 113.675 73.525) (end 113.925 73.275) (width 0.2) (layer "B.Cu") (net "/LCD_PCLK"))
 (segment (start 113.925 73.275) (end 113.925 63.75) (width 0.2) (layer "B.Cu") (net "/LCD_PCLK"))
 (segment (start 112.625 62.45) (end 113.925 63.75) (width 0.2) (layer "B.Cu") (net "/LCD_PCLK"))
 (segment (start 100.45 77.175) (end 100.45 74) (width 0.2) (layer "F.Cu") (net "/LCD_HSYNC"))
 (segment (start 99.95 73.5) (end 100.45 74) (width 0.2) (layer "F.Cu") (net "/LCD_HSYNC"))
 (segment (start 99.95 65.675) (end 99.95 73.5) (width 0.2) (layer "F.Cu") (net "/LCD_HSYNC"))
 (segment (start 99.95 77.175) (end 99.95 74.065686) (width 0.2) (layer "F.Cu") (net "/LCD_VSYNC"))
 (segment (start 99.45 65.675) (end 99.45 73.565686) (width 0.2) (layer "F.Cu") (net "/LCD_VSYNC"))
 (segment (start 99.95 74.065686) (end 99.45 73.565686) (width 0.2) (layer "F.Cu") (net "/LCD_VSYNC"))
 (segment (start 98.95 73.675) (end 99.45 74.175) (width 0.2) (layer "F.Cu") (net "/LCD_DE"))
 (segment (start 99.45 77.175) (end 99.45 74.175) (width 0.2) (layer "F.Cu") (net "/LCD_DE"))
 (segment (start 98.95 65.675) (end 98.95 73.675) (width 0.2) (layer "F.Cu") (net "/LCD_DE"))
 (segment (start 97.95 72.05) (end 96.45 73.55) (width 0.2) (layer "F.Cu") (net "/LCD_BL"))
 (segment (start 96.45 77.175) (end 96.45 73.55) (width 0.2) (layer "F.Cu") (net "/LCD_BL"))
 (segment (start 97.95 65.675) (end 97.95 72.05) (width 0.2) (layer "F.Cu") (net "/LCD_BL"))
 (segment (start 98.95 77.175) (end 98.95 78.875) (width 0.2) (layer "F.Cu") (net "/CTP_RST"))
 (segment (start 96.95 65.675) (end 96.95 63.951471) (width 0.2) (layer "F.Cu") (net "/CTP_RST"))
 (segment (start 97.676471 63.225) (end 98.725 63.225) (width 0.2) (layer "F.Cu") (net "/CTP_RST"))
 (segment (start 96.95 63.951471) (end 97.676471 63.225) (width 0.2) (layer "F.Cu") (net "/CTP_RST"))
 (segment (start 98.725 63.225) (end 99.325 62.625) (width 0.2) (layer "F.Cu") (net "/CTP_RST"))
 (via (at 99.325 62.625) (size 0.6) (drill 0.3) (layers "F.Cu" "B.Cu") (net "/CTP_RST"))
 (via (at 98.95 78.875) (size 0.6) (drill 0.3) (layers "F.Cu" "B.Cu") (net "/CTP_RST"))
 (segment (start 98.95 78.875) (end 99.325 78.5) (width 0.2) (layer "B.Cu") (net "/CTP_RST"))
 (segment (start 99.325 62.625) (end 99.325 78.5) (width 0.2) (layer "B.Cu") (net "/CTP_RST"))
 (segment (start 113.95 78.85) (end 113.95 77.175) (width 0.2) (layer "F.Cu") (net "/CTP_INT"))
 (segment (start 112.15 80.65) (end 113.95 78.85) (width 0.2) (layer "F.Cu") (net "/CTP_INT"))
 (segment (start 96.45 69.025) (end 96.45 65.675) (width 0.2) (layer "F.Cu") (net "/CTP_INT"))
 (via (at 112.15 80.65) (size 0.6) (drill 0.3) (layers "F.Cu" "B.Cu") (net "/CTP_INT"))
 (via (at 96.45 69.025) (size 0.6) (drill 0.3) (layers "F.Cu" "B.Cu") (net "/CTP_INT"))
 (segment (start 96.45 69.025) (end 96.45 78.375) (width 0.2) (layer "B.Cu") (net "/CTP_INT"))
 (segment (start 98.725 80.65) (end 112.15 80.65) (width 0.2) (layer "B.Cu") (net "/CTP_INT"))
 (segment (start 96.45 78.375) (end 98.725 80.65) (width 0.2) (layer "B.Cu") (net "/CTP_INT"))
 (segment (start 110.275 81.275) (end 111.625 81.275) (width 0.2) (layer "F.Cu") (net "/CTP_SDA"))
 (segment (start 114.975 81.25) (end 114.95 81.225) (width 0.2) (layer "F.Cu") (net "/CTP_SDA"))
 (segment (start 112.925 82.575) (end 114.2 82.575) (width 0.2) (layer "F.Cu") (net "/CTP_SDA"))
 (segment (start 95.653601 68.97287) (end 95.95 68.676471) (width 0.2) (layer "F.Cu") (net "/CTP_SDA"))
 (segment (start 114.95 81.225) (end 114.95 77.175) (width 0.2) (layer "F.Cu") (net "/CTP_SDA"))
 (segment (start 95.653601 69.100848) (end 95.653601 68.97287) (width 0.2) (layer "F.Cu") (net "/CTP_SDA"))
 (segment (start 114.2 82.575) (end 114.975 81.8) (width 0.2) (layer "F.Cu") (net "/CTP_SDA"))
 (segment (start 114.975 81.8) (end 114.975 81.25) (width 0.2) (layer "F.Cu") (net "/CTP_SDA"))
 (segment (start 95.95 68.676471) (end 95.95 65.675) (width 0.2) (layer "F.Cu") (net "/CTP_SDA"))
 (segment (start 111.625 81.275) (end 112.925 82.575) (width 0.2) (layer "F.Cu") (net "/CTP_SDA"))
 (via (at 110.275 81.275) (size 0.6) (drill 0.3) (layers "F.Cu" "B.Cu") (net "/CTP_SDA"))
 (via (at 95.653601 69.100848) (size 0.6) (drill 0.3) (layers "F.Cu" "B.Cu") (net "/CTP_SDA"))
 (segment (start 98.303601 81.275) (end 110.275 81.275) (width 0.2) (layer "B.Cu") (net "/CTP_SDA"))
 (segment (start 95.653601 78.625) (end 98.303601 81.275) (width 0.2) (layer "B.Cu") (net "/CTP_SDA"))
 (segment (start 95.653601 69.100848) (end 95.653601 78.625) (width 0.2) (layer "B.Cu") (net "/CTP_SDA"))
 (segment (start 114.45 80.025) (end 114.45 77.175) (width 0.2) (layer "F.Cu") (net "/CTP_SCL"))
 (segment (start 95.45 68.45592) (end 95.45 65.675) (width 0.2) (layer "F.Cu") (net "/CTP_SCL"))
 (segment (start 113.6 80.875) (end 114.45 80.025) (width 0.2) (layer "F.Cu") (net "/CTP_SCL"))
 (segment (start 94.85 69.05592) (end 95.45 68.45592) (width 0.2) (layer "F.Cu") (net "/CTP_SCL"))
 (segment (start 94.85 69.075) (end 94.85 69.05592) (width 0.2) (layer "F.Cu") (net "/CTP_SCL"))
 (via (at 94.85 69.075) (size 0.6) (drill 0.3) (layers "F.Cu" "B.Cu") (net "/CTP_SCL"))
 (via (at 113.6 80.875) (size 0.6) (drill 0.3) (layers "F.Cu" "B.Cu") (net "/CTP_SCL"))
 (segment (start 94.85 78.875) (end 97.85 81.875) (width 0.2) (layer "B.Cu") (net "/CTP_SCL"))
 (segment (start 94.85 78.875) (end 94.85 69.075) (width 0.2) (layer "B.Cu") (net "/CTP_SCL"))
 (segment (start 112.6 81.875) (end 113.6 80.875) (width 0.2) (layer "B.Cu") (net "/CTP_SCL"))
 (segment (start 97.85 81.875) (end 112.6 81.875) (width 0.2) (layer "B.Cu") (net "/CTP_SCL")))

